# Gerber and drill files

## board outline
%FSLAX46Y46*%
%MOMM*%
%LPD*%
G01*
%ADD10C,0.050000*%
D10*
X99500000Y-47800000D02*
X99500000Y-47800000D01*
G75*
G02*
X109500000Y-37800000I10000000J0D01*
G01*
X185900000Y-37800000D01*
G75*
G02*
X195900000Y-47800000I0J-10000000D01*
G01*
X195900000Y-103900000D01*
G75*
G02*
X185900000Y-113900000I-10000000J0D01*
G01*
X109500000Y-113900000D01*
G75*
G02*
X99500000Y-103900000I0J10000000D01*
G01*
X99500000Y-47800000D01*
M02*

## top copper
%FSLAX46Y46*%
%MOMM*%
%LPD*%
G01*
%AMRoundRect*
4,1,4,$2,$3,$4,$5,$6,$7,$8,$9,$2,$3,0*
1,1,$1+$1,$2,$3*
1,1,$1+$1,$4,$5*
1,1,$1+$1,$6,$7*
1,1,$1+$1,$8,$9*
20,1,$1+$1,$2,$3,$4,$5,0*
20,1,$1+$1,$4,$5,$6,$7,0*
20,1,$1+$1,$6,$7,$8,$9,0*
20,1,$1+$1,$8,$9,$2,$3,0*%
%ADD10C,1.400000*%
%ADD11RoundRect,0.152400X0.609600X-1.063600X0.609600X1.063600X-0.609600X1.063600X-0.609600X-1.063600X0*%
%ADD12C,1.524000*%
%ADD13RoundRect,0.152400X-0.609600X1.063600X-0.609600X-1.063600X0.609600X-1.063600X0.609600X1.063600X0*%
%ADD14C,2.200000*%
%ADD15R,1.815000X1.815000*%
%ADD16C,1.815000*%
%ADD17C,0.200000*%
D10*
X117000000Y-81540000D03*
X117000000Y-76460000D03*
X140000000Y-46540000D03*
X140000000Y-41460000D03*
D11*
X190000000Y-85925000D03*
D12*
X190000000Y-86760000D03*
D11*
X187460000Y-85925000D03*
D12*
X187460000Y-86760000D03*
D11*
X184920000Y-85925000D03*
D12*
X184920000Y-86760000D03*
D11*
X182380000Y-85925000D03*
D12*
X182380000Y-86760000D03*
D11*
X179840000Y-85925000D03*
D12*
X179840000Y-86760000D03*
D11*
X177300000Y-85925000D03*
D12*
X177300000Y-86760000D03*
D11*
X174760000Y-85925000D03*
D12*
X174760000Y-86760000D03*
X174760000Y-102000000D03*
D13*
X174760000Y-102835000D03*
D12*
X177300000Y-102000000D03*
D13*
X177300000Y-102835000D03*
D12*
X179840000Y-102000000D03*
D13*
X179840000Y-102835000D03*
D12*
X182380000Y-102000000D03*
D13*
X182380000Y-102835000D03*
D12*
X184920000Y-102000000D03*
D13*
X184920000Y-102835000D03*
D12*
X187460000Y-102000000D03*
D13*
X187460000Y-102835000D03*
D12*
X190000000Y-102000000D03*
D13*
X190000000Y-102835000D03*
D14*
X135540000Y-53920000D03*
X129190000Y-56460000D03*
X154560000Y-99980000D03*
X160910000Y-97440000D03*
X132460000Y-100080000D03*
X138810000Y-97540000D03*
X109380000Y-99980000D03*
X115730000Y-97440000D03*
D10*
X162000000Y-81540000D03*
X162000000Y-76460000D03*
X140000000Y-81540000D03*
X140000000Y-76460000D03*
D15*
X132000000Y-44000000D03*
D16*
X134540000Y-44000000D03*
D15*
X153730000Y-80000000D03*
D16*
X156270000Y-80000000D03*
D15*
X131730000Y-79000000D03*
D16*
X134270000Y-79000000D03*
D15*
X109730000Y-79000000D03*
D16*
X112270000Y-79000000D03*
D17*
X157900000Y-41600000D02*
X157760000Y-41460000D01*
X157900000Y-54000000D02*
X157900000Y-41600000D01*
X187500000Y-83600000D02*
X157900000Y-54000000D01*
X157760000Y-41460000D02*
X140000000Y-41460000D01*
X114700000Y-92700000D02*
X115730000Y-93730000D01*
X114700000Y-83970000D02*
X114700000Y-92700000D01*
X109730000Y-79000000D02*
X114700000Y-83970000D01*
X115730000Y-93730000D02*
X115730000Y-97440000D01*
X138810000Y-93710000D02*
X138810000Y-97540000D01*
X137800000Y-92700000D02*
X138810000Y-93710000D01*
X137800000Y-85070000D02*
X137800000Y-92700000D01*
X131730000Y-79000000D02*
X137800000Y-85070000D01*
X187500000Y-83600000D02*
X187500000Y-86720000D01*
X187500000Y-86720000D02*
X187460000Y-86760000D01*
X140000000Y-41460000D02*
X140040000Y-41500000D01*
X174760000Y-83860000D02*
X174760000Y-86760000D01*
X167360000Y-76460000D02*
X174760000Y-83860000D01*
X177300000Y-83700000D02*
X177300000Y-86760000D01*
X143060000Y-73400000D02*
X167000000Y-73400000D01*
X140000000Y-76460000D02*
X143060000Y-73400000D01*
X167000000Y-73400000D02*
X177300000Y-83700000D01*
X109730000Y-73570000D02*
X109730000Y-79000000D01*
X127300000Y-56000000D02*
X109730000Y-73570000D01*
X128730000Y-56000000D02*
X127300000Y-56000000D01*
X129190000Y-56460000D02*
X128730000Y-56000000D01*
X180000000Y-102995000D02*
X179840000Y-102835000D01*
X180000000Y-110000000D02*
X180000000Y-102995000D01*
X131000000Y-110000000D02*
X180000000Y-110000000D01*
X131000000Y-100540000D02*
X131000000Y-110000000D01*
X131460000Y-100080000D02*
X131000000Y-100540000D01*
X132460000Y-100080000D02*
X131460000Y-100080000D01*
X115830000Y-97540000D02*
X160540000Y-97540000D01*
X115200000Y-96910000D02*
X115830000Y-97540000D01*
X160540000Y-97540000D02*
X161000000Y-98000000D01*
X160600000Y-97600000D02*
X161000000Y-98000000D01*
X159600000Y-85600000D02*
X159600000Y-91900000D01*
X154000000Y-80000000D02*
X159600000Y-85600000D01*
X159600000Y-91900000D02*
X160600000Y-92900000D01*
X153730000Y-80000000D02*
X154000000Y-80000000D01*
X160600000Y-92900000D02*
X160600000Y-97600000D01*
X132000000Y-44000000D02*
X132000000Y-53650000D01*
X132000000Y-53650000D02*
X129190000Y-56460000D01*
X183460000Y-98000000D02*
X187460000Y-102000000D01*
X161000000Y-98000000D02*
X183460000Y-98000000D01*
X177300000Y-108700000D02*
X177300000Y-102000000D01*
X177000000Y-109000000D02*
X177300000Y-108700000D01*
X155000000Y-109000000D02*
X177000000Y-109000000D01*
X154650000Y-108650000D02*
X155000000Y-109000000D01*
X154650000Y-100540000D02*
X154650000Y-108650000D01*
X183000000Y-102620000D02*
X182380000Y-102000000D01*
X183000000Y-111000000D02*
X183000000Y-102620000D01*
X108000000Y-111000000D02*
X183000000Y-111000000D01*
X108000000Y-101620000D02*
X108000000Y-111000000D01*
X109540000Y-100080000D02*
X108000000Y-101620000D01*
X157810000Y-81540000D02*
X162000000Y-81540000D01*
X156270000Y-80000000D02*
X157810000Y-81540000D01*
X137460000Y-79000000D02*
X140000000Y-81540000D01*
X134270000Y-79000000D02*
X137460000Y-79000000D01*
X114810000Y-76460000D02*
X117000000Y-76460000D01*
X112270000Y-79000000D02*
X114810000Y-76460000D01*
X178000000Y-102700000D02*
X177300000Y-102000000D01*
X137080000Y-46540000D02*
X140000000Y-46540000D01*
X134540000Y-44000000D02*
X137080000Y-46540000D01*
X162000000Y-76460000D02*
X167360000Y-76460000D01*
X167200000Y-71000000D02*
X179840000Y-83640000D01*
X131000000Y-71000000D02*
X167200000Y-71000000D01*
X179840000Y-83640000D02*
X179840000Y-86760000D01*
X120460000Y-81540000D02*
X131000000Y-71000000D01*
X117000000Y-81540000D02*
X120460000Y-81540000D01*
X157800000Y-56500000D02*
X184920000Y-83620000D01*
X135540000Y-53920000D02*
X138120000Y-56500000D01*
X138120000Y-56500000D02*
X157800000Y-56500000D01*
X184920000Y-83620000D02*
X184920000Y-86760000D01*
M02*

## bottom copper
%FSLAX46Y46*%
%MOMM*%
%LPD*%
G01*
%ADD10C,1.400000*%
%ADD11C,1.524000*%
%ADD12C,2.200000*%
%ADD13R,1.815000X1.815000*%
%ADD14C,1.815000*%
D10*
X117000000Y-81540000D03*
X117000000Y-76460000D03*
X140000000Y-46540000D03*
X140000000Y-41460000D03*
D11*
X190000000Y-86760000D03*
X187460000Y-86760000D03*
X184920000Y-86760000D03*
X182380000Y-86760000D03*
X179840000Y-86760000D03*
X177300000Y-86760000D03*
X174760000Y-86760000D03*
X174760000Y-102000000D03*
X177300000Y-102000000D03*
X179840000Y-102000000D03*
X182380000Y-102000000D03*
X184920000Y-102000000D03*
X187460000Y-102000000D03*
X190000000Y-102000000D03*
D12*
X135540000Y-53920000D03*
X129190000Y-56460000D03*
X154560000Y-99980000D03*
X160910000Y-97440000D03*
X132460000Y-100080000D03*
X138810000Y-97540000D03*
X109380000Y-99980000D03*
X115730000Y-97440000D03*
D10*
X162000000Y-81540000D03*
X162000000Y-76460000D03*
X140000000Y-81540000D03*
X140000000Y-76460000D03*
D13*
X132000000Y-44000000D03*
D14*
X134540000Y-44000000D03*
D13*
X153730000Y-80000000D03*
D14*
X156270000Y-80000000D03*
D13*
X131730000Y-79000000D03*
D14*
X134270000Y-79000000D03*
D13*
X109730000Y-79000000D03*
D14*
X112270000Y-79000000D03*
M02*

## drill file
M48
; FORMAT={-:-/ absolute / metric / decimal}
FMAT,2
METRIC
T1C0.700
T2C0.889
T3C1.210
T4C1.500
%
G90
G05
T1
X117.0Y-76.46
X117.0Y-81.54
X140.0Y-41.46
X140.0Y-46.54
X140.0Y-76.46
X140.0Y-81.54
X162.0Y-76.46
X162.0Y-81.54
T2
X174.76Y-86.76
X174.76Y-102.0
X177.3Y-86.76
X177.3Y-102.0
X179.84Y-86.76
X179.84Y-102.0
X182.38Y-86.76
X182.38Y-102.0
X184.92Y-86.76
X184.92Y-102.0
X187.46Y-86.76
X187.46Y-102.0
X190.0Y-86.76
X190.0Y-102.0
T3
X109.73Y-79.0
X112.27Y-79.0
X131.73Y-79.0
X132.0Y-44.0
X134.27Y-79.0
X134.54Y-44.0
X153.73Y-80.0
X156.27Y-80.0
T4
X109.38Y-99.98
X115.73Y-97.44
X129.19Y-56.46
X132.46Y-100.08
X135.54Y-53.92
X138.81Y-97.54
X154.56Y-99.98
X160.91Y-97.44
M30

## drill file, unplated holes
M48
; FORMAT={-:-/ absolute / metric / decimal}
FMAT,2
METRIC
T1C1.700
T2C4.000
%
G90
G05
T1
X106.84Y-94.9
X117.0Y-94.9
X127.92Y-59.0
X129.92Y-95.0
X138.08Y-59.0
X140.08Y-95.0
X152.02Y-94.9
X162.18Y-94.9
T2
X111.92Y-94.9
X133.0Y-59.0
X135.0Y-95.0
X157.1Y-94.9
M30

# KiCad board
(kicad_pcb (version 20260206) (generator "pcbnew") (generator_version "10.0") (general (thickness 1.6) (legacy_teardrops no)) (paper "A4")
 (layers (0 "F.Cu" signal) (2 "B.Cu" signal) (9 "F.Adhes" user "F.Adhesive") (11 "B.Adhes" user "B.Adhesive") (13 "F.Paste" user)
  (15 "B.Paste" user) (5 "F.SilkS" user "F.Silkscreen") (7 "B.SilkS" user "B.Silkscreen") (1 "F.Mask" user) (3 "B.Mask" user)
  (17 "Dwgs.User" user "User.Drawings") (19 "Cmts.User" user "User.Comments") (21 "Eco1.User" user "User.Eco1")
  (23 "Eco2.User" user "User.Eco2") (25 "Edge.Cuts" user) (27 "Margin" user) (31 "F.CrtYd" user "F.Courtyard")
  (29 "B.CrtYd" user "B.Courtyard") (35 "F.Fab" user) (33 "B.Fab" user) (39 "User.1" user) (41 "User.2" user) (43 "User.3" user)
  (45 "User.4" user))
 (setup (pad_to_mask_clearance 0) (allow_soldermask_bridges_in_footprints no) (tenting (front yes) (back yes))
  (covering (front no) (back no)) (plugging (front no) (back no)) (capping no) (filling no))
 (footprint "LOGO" (layer "F.Cu") (at 111.4 50.9)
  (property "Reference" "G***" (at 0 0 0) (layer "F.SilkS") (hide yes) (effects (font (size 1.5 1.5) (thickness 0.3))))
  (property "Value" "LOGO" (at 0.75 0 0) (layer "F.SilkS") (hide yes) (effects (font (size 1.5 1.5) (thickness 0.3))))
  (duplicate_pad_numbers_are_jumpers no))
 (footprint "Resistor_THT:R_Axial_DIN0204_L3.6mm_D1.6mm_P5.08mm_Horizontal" (layer "F.Cu") (at 140 46.54 90)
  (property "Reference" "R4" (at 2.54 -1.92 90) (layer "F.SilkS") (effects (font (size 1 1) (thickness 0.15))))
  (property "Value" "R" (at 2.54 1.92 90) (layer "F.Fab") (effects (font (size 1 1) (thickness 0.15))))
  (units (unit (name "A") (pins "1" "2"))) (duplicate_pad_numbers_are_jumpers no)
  (pad "1" thru_hole circle (at 0 0 90) (size 1.4 1.4) (drill 0.7) (layers "*.Cu" "*.Mask") (remove_unused_layers no) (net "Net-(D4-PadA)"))
  (pad "2" thru_hole circle (at 5.08 0 90) (size 1.4 1.4) (drill 0.7) (layers "*.Cu" "*.Mask") (remove_unused_layers no) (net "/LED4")))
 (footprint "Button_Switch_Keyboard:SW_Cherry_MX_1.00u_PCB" (layer "F.Cu") (at 154.56 99.98 180)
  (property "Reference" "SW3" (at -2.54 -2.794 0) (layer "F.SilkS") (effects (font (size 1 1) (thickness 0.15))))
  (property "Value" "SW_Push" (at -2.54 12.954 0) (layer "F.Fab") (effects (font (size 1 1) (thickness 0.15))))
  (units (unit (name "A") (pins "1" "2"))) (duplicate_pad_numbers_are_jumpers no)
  (pad "" np_thru_hole circle (at -7.62 5.08 180) (size 1.7 1.7) (drill 1.7) (layers "*.Cu" "*.Mask"))
  (pad "" np_thru_hole circle (at -2.54 5.08 180) (size 4 4) (drill 4) (layers "*.Cu" "*.Mask"))
  (pad "" np_thru_hole circle (at 2.54 5.08 180) (size 1.7 1.7) (drill 1.7) (layers "*.Cu" "*.Mask"))
  (pad "1" thru_hole circle (at 0 0 180) (size 2.2 2.2) (drill 1.5) (layers "*.Cu" "*.Mask") (remove_unused_layers no) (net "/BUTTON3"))
  (pad "2" thru_hole circle (at -6.35 2.54 180) (size 2.2 2.2) (drill 1.5) (layers "*.Cu" "*.Mask") (remove_unused_layers no) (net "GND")))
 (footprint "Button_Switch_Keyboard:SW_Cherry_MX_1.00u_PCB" (layer "F.Cu") (at 132.46 100.08 180)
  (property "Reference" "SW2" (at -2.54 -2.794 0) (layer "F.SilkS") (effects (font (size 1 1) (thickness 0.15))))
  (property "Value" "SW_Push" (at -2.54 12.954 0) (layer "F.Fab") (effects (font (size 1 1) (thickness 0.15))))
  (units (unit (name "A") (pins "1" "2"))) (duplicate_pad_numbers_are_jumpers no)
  (pad "" np_thru_hole circle (at -7.62 5.08 180) (size 1.7 1.7) (drill 1.7) (layers "*.Cu" "*.Mask"))
  (pad "" np_thru_hole circle (at -2.54 5.08 180) (size 4 4) (drill 4) (layers "*.Cu" "*.Mask"))
  (pad "" np_thru_hole circle (at 2.54 5.08 180) (size 1.7 1.7) (drill 1.7) (layers "*.Cu" "*.Mask"))
  (pad "1" thru_hole circle (at 0 0 180) (size 2.2 2.2) (drill 1.5) (layers "*.Cu" "*.Mask") (remove_unused_layers no) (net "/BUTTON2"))
  (pad "2" thru_hole circle (at -6.35 2.54 180) (size 2.2 2.2) (drill 1.5) (layers "*.Cu" "*.Mask") (remove_unused_layers no) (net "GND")))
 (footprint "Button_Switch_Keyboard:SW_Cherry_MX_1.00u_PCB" (layer "F.Cu") (at 135.54 53.92)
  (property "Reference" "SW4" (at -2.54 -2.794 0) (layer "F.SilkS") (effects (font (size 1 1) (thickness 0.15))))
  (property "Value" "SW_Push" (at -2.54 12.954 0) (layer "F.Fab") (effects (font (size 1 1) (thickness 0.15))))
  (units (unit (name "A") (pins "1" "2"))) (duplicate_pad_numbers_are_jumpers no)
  (pad "" np_thru_hole circle (at -7.62 5.08) (size 1.7 1.7) (drill 1.7) (layers "*.Cu" "*.Mask"))
  (pad "" np_thru_hole circle (at -2.54 5.08) (size 4 4) (drill 4) (layers "*.Cu" "*.Mask"))
  (pad "" np_thru_hole circle (at 2.54 5.08) (size 1.7 1.7) (drill 1.7) (layers "*.Cu" "*.Mask"))
  (pad "1" thru_hole circle (at 0 0) (size 2.2 2.2) (drill 1.5) (layers "*.Cu" "*.Mask") (remove_unused_layers no) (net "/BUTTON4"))
  (pad "2" thru_hole circle (at -6.35 2.54) (size 2.2 2.2) (drill 1.5) (layers "*.Cu" "*.Mask") (remove_unused_layers no) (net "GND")))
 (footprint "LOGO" (layer "F.Cu") (at 180.3 64.4)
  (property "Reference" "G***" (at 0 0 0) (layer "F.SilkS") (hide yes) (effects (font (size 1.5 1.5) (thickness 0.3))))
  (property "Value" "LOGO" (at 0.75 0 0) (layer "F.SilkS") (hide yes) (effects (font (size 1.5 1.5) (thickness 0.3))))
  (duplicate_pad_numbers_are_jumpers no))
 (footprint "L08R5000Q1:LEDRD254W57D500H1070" (layer "F.Cu") (at 133.27 44)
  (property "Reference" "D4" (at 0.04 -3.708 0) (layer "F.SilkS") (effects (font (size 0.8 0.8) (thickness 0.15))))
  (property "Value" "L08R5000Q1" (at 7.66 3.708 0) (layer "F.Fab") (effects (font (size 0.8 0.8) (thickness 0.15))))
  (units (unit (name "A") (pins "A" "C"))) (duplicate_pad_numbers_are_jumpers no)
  (pad "A" thru_hole circle (at 1.27 0) (size 1.815 1.815) (drill 1.21) (layers "*.Cu" "*.Mask") (remove_unused_layers no)
   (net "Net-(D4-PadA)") (solder_mask_margin 0.102))
  (pad "C" thru_hole rect (at -1.27 0) (size 1.815 1.815) (drill 1.21) (layers "*.Cu" "*.Mask") (remove_unused_layers no) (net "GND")
   (solder_mask_margin 0.102)))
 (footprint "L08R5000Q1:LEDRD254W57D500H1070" (layer "F.Cu") (at 155 80)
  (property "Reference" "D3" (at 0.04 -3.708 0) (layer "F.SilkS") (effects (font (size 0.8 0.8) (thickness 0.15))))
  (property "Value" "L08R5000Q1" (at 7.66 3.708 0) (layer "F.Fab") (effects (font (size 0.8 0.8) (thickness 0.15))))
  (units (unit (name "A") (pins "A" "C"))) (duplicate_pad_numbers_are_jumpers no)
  (pad "A" thru_hole circle (at 1.27 0) (size 1.815 1.815) (drill 1.21) (layers "*.Cu" "*.Mask") (remove_unused_layers no)
   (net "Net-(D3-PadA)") (solder_mask_margin 0.102))
  (pad "C" thru_hole rect (at -1.27 0) (size 1.815 1.815) (drill 1.21) (layers "*.Cu" "*.Mask") (remove_unused_layers no) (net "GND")
   (solder_mask_margin 0.102)))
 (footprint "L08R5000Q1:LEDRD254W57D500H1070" (layer "F.Cu") (at 111 79)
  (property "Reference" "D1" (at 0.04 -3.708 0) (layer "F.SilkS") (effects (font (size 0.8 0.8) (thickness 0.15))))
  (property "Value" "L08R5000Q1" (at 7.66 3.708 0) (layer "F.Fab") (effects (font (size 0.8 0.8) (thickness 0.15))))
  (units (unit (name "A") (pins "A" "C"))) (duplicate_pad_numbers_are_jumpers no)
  (pad "A" thru_hole circle (at 1.27 0) (size 1.815 1.815) (drill 1.21) (layers "*.Cu" "*.Mask") (remove_unused_layers no)
   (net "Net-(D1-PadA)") (solder_mask_margin 0.102))
  (pad "C" thru_hole rect (at -1.27 0) (size 1.815 1.815) (drill 1.21) (layers "*.Cu" "*.Mask") (remove_unused_layers no) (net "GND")
   (solder_mask_margin 0.102)))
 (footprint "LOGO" (layer "F.Cu") (at 170.3 47.5)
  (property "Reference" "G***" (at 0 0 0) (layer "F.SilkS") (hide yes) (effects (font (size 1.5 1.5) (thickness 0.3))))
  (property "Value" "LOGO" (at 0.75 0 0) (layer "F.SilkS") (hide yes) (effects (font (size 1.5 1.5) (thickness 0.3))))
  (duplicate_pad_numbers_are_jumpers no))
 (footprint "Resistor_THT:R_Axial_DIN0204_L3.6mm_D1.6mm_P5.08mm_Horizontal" (layer "F.Cu") (at 117 81.54 90)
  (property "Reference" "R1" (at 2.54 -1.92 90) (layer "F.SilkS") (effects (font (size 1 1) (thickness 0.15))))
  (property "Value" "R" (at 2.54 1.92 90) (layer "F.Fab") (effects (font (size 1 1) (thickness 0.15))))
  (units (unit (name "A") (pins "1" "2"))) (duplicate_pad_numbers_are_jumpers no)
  (pad "1" thru_hole circle (at 0 0 90) (size 1.4 1.4) (drill 0.7) (layers "*.Cu" "*.Mask") (remove_unused_layers no) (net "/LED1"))
  (pad "2" thru_hole circle (at 5.08 0 90) (size 1.4 1.4) (drill 0.7) (layers "*.Cu" "*.Mask") (remove_unused_layers no)
   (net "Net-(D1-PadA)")))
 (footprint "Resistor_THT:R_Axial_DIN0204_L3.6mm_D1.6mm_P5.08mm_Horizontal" (layer "F.Cu") (at 162 81.54 90)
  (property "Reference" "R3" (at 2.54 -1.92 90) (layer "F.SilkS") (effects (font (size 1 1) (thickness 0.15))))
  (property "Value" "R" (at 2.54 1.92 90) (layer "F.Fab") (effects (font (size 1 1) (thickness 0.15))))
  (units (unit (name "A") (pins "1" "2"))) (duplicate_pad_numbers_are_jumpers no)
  (pad "1" thru_hole circle (at 0 0 90) (size 1.4 1.4) (drill 0.7) (layers "*.Cu" "*.Mask") (remove_unused_layers no) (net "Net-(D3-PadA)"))
  (pad "2" thru_hole circle (at 5.08 0 90) (size 1.4 1.4) (drill 0.7) (layers "*.Cu" "*.Mask") (remove_unused_layers no) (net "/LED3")))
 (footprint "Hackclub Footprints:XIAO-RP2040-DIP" (layer "F.Cu") (at 182.38 94.38 -90)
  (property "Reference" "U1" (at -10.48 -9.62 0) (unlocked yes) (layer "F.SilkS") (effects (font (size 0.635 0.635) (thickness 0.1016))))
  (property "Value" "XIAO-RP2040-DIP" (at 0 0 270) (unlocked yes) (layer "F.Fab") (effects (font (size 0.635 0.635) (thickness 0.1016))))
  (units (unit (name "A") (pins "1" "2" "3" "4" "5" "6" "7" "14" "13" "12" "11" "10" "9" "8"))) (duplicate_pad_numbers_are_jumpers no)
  (pad "1" smd roundrect (at -8.455 -7.62 90) (size 2.432 1.524) (layers "F.Cu" "F.Mask") (roundrect_rratio 0.1)
   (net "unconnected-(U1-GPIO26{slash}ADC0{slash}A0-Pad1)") (thermal_bridge_angle 45))
  (pad "1" thru_hole circle (at -7.62 -7.62 90) (size 1.524 1.524) (drill 0.889) (layers "*.Cu" "*.Mask") (remove_unused_layers no)
   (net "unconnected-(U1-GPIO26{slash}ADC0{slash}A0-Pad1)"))
  (pad "2" smd roundrect (at -8.455 -5.08 90) (size 2.432 1.524) (layers "F.Cu" "F.Mask") (roundrect_rratio 0.1) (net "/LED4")
   (thermal_bridge_angle 45))
  (pad "2" thru_hole circle (at -7.62 -5.08 90) (size 1.524 1.524) (drill 0.889) (layers "*.Cu" "*.Mask") (remove_unused_layers no)
   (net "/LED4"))
  (pad "3" smd roundrect (at -8.455 -2.54 90) (size 2.432 1.524) (layers "F.Cu" "F.Mask") (roundrect_rratio 0.1) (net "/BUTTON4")
   (thermal_bridge_angle 45))
  (pad "3" thru_hole circle (at -7.62 -2.54 90) (size 1.524 1.524) (drill 0.889) (layers "*.Cu" "*.Mask") (remove_unused_layers no)
   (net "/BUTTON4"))
  (pad "4" smd roundrect (at -8.455 0 90) (size 2.432 1.524) (layers "F.Cu" "F.Mask") (roundrect_rratio 0.1)
   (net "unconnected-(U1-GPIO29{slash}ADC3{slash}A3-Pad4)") (thermal_bridge_angle 45))
  (pad "4" thru_hole circle (at -7.62 0 90) (size 1.524 1.524) (drill 0.889) (layers "*.Cu" "*.Mask") (remove_unused_layers no)
   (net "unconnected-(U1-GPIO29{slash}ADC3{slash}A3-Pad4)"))
  (pad "5" smd roundrect (at -8.455 2.54 90) (size 2.432 1.524) (layers "F.Cu" "F.Mask") (roundrect_rratio 0.1) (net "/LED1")
   (thermal_bridge_angle 45))
  (pad "5" thru_hole circle (at -7.62 2.54 90) (size 1.524 1.524) (drill 0.889) (layers "*.Cu" "*.Mask") (remove_unused_layers no)
   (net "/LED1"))
  (pad "6" smd roundrect (at -8.455 5.08 90) (size 2.432 1.524) (layers "F.Cu" "F.Mask") (roundrect_rratio 0.1) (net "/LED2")
   (thermal_bridge_angle 45))
  (pad "6" thru_hole circle (at -7.62 5.08 90) (size 1.524 1.524) (drill 0.889) (layers "*.Cu" "*.Mask") (remove_unused_layers no)
   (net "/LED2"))
  (pad "7" smd roundrect (at -8.455 7.62 90) (size 2.432 1.524) (layers "F.Cu" "F.Mask") (roundrect_rratio 0.1) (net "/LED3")
   (thermal_bridge_angle 45))
  (pad "7" thru_hole circle (at -7.62 7.62 90) (size 1.524 1.524) (drill 0.889) (layers "*.Cu" "*.Mask") (remove_unused_layers no)
   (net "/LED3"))
  (pad "8" thru_hole circle (at 7.62 7.62 270) (size 1.524 1.524) (drill 0.889) (layers "*.Cu" "*.Mask") (remove_unused_layers no)
   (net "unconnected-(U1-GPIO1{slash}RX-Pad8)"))
  (pad "8" smd roundrect (at 8.455 7.62 270) (size 2.432 1.524) (layers "F.Cu" "F.Mask") (roundrect_rratio 0.1)
   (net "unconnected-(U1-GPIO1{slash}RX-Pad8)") (thermal_bridge_angle 45))
  (pad "9" thru_hole circle (at 7.62 5.08 270) (size 1.524 1.524) (drill 0.889) (layers "*.Cu" "*.Mask") (remove_unused_layers no)
   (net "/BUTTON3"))
  (pad "9" smd roundrect (at 8.455 5.08 270) (size 2.432 1.524) (layers "F.Cu" "F.Mask") (roundrect_rratio 0.1) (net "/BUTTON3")
   (thermal_bridge_angle 45))
  (pad "10" thru_hole circle (at 7.62 2.54 270) (size 1.524 1.524) (drill 0.889) (layers "*.Cu" "*.Mask") (remove_unused_layers no)
   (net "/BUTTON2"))
  (pad "10" smd roundrect (at 8.455 2.54 270) (size 2.432 1.524) (layers "F.Cu" "F.Mask") (roundrect_rratio 0.1) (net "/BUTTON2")
   (thermal_bridge_angle 45))
  (pad "11" thru_hole circle (at 7.62 0 270) (size 1.524 1.524) (drill 0.889) (layers "*.Cu" "*.Mask") (remove_unused_layers no)
   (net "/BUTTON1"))
  (pad "11" smd roundrect (at 8.455 0 270) (size 2.432 1.524) (layers "F.Cu" "F.Mask") (roundrect_rratio 0.1) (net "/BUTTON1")
   (thermal_bridge_angle 45))
  (pad "12" thru_hole circle (at 7.62 -2.54 270) (size 1.524 1.524) (drill 0.889) (layers "*.Cu" "*.Mask") (remove_unused_layers no)
   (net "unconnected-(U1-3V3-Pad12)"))
  (pad "12" smd roundrect (at 8.455 -2.54 270) (size 2.432 1.524) (layers "F.Cu" "F.Mask") (roundrect_rratio 0.1)
   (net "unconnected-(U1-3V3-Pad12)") (thermal_bridge_angle 45))
  (pad "13" thru_hole circle (at 7.62 -5.08 270) (size 1.524 1.524) (drill 0.889) (layers "*.Cu" "*.Mask") (remove_unused_layers no)
   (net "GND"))
  (pad "13" smd roundrect (at 8.455 -5.08 270) (size 2.432 1.524) (layers "F.Cu" "F.Mask") (roundrect_rratio 0.1) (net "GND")
   (thermal_bridge_angle 45))
  (pad "14" thru_hole circle (at 7.62 -7.62 270) (size 1.524 1.524) (drill 0.889) (layers "*.Cu" "*.Mask") (remove_unused_layers no)
   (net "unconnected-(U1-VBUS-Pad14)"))
  (pad "14" smd roundrect (at 8.455 -7.62 270) (size 2.432 1.524) (layers "F.Cu" "F.Mask") (roundrect_rratio 0.1)
   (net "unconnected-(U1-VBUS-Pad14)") (thermal_bridge_angle 45)))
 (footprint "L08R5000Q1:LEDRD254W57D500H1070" (layer "F.Cu") (at 133 79)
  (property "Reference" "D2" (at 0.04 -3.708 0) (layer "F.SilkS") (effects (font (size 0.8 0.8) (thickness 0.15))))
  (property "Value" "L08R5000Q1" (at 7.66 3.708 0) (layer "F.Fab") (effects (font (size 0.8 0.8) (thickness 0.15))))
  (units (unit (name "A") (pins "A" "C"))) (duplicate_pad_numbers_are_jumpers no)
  (pad "A" thru_hole circle (at 1.27 0) (size 1.815 1.815) (drill 1.21) (layers "*.Cu" "*.Mask") (remove_unused_layers no)
   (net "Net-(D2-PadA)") (solder_mask_margin 0.102))
  (pad "C" thru_hole rect (at -1.27 0) (size 1.815 1.815) (drill 1.21) (layers "*.Cu" "*.Mask") (remove_unused_layers no) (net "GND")
   (solder_mask_margin 0.102)))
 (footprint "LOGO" (layer "F.Cu") (at 182.9 51.3)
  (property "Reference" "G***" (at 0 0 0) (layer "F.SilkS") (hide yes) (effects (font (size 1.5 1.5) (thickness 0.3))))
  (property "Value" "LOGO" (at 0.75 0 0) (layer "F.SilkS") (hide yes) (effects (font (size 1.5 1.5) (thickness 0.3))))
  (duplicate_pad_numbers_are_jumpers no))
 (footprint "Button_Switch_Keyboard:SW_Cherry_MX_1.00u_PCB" (layer "F.Cu") (at 109.38 99.98 180)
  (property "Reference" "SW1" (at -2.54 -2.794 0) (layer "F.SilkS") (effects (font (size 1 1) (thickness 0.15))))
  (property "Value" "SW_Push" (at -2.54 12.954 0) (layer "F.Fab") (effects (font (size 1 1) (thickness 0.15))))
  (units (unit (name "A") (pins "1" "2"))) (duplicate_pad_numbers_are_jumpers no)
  (pad "" np_thru_hole circle (at -7.62 5.08 180) (size 1.7 1.7) (drill 1.7) (layers "*.Cu" "*.Mask"))
  (pad "" np_thru_hole circle (at -2.54 5.08 180) (size 4 4) (drill 4) (layers "*.Cu" "*.Mask"))
  (pad "" np_thru_hole circle (at 2.54 5.08 180) (size 1.7 1.7) (drill 1.7) (layers "*.Cu" "*.Mask"))
  (pad "1" thru_hole circle (at 0 0 180) (size 2.2 2.2) (drill 1.5) (layers "*.Cu" "*.Mask") (remove_unused_layers no) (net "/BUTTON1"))
  (pad "2" thru_hole circle (at -6.35 2.54 180) (size 2.2 2.2) (drill 1.5) (layers "*.Cu" "*.Mask") (remove_unused_layers no) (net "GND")))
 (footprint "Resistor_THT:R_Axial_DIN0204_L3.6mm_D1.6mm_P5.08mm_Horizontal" (layer "F.Cu") (at 140 81.54 90)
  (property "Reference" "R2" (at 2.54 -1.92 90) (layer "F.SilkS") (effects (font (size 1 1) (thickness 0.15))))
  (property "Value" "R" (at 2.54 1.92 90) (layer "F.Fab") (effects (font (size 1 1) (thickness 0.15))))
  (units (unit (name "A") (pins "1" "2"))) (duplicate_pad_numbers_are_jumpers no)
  (pad "1" thru_hole circle (at 0 0 90) (size 1.4 1.4) (drill 0.7) (layers "*.Cu" "*.Mask") (remove_unused_layers no) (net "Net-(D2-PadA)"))
  (pad "2" thru_hole circle (at 5.08 0 90) (size 1.4 1.4) (drill 0.7) (layers "*.Cu" "*.Mask") (remove_unused_layers no) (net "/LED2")))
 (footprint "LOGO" (layer "B.Cu") (at 179.405448 56.483194 180)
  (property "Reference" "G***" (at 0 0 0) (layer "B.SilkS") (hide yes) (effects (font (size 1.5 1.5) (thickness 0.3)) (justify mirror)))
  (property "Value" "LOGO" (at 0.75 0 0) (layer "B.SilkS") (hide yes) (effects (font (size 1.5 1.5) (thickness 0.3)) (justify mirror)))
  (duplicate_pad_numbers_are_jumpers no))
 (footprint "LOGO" (layer "B.Cu") (at 110.818051 63.678154 180)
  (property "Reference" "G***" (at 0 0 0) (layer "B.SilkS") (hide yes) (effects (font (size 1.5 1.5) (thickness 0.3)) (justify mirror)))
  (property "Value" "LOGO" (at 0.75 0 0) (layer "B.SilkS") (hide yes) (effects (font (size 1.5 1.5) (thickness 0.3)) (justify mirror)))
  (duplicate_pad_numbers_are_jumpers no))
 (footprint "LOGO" (layer "B.Cu") (at 111.204014 47.294564 180)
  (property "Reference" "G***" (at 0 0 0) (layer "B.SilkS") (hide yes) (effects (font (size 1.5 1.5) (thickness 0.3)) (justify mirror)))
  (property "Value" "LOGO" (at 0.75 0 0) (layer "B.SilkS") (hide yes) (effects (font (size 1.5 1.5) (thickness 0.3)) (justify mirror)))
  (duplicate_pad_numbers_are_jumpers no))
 (gr_rect (start 99.5 37.8) (end 195.9 113.9) (radius 10) (stroke (width 0.05) (type solid)) (fill no) (layer "Edge.Cuts"))
 (segment (start 114.81 76.46) (end 117 76.46) (width 0.2) (layer "F.Cu") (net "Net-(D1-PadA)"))
 (segment (start 112.27 79) (end 114.81 76.46) (width 0.2) (layer "F.Cu") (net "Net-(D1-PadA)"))
 (segment (start 138.81 93.71) (end 138.81 97.54) (width 0.2) (layer "F.Cu") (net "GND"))
 (segment (start 115.73 93.73) (end 115.73 97.44) (width 0.2) (layer "F.Cu") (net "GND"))
 (segment (start 183.46 98) (end 187.46 102) (width 0.2) (layer "F.Cu") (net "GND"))
 (segment (start 159.6 91.9) (end 160.6 92.9) (width 0.2) (layer "F.Cu") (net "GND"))
 (segment (start 160.6 92.9) (end 160.6 97.6) (width 0.2) (layer "F.Cu") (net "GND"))
 (segment (start 132 44) (end 132 53.65) (width 0.2) (layer "F.Cu") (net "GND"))
 (segment (start 154 80) (end 159.6 85.6) (width 0.2) (layer "F.Cu") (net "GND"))
 (segment (start 129.19 56.46) (end 128.73 56) (width 0.2) (layer "F.Cu") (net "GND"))
 (segment (start 115.2 96.91) (end 115.83 97.54) (width 0.2) (layer "F.Cu") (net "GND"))
 (segment (start 153.73 80) (end 154 80) (width 0.2) (layer "F.Cu") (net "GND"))
 (segment (start 109.73 73.57) (end 109.73 79) (width 0.2) (layer "F.Cu") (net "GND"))
 (segment (start 128.73 56) (end 127.3 56) (width 0.2) (layer "F.Cu") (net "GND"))
 (segment (start 114.7 83.97) (end 114.7 92.7) (width 0.2) (layer "F.Cu") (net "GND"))
 (segment (start 160.54 97.54) (end 161 98) (width 0.2) (layer "F.Cu") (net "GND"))
 (segment (start 159.6 85.6) (end 159.6 91.9) (width 0.2) (layer "F.Cu") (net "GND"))
 (segment (start 109.73 79) (end 114.7 83.97) (width 0.2) (layer "F.Cu") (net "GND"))
 (segment (start 131.73 79) (end 137.8 85.07) (width 0.2) (layer "F.Cu") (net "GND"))
 (segment (start 137.8 92.7) (end 138.81 93.71) (width 0.2) (layer "F.Cu") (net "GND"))
 (segment (start 114.7 92.7) (end 115.73 93.73) (width 0.2) (layer "F.Cu") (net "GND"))
 (segment (start 127.3 56) (end 109.73 73.57) (width 0.2) (layer "F.Cu") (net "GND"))
 (segment (start 160.6 97.6) (end 161 98) (width 0.2) (layer "F.Cu") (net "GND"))
 (segment (start 161 98) (end 183.46 98) (width 0.2) (layer "F.Cu") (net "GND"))
 (segment (start 132 53.65) (end 129.19 56.46) (width 0.2) (layer "F.Cu") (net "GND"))
 (segment (start 115.83 97.54) (end 160.54 97.54) (width 0.2) (layer "F.Cu") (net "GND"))
 (segment (start 137.8 85.07) (end 137.8 92.7) (width 0.2) (layer "F.Cu") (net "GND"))
 (segment (start 137.46 79) (end 140 81.54) (width 0.2) (layer "F.Cu") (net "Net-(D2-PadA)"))
 (segment (start 134.27 79) (end 137.46 79) (width 0.2) (layer "F.Cu") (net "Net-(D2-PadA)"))
 (segment (start 157.81 81.54) (end 162 81.54) (width 0.2) (layer "F.Cu") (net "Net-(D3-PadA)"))
 (segment (start 156.27 80) (end 157.81 81.54) (width 0.2) (layer "F.Cu") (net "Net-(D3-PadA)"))
 (segment (start 134.54 44) (end 137.08 46.54) (width 0.2) (layer "F.Cu") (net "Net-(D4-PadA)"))
 (segment (start 137.08 46.54) (end 140 46.54) (width 0.2) (layer "F.Cu") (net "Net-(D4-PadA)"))
 (segment (start 167.2 71) (end 179.84 83.64) (width 0.2) (layer "F.Cu") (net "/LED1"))
 (segment (start 131 71) (end 167.2 71) (width 0.2) (layer "F.Cu") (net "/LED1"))
 (segment (start 117 81.54) (end 120.46 81.54) (width 0.2) (layer "F.Cu") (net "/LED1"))
 (segment (start 179.84 83.64) (end 179.84 86.76) (width 0.2) (layer "F.Cu") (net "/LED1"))
 (segment (start 120.46 81.54) (end 131 71) (width 0.2) (layer "F.Cu") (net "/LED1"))
 (segment (start 140 76.46) (end 143.06 73.4) (width 0.2) (layer "F.Cu") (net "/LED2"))
 (segment (start 143.06 73.4) (end 167 73.4) (width 0.2) (layer "F.Cu") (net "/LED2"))
 (segment (start 177.3 83.7) (end 177.3 86.76) (width 0.2) (layer "F.Cu") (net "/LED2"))
 (segment (start 167 73.4) (end 177.3 83.7) (width 0.2) (layer "F.Cu") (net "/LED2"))
 (segment (start 162 76.46) (end 167.36 76.46) (width 0.2) (layer "F.Cu") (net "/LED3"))
 (segment (start 167.36 76.46) (end 174.76 83.86) (width 0.2) (layer "F.Cu") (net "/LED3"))
 (segment (start 174.76 83.86) (end 174.76 86.76) (width 0.2) (layer "F.Cu") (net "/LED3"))
 (segment (start 187.5 83.6) (end 187.5 86.72) (width 0.2) (layer "F.Cu") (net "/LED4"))
 (segment (start 187.5 83.6) (end 157.9 54) (width 0.2) (layer "F.Cu") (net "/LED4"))
 (segment (start 187.5 86.72) (end 187.46 86.76) (width 0.2) (layer "F.Cu") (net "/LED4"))
 (segment (start 140 41.46) (end 140.04 41.5) (width 0.2) (layer "F.Cu") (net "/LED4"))
 (segment (start 157.9 41.6) (end 157.76 41.46) (width 0.2) (layer "F.Cu") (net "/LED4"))
 (segment (start 157.76 41.46) (end 140 41.46) (width 0.2) (layer "F.Cu") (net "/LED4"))
 (segment (start 157.9 54) (end 157.9 41.6) (width 0.2) (layer "F.Cu") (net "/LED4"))
 (segment (start 109.54 100.08) (end 108 101.62) (width 0.2) (layer "F.Cu") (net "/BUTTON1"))
 (segment (start 108 101.62) (end 108 111) (width 0.2) (layer "F.Cu") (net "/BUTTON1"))
 (segment (start 108 111) (end 183 111) (width 0.2) (layer "F.Cu") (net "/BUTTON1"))
 (segment (start 183 102.62) (end 182.38 102) (width 0.2) (layer "F.Cu") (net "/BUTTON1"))
 (segment (start 183 111) (end 183 102.62) (width 0.2) (layer "F.Cu") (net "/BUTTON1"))
 (segment (start 131 110) (end 180 110) (width 0.2) (layer "F.Cu") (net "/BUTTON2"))
 (segment (start 131.46 100.08) (end 131 100.54) (width 0.2) (layer "F.Cu") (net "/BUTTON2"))
 (segment (start 131 100.54) (end 131 110) (width 0.2) (layer "F.Cu") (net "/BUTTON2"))
 (segment (start 132.46 100.08) (end 131.46 100.08) (width 0.2) (layer "F.Cu") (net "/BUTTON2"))
 (segment (start 180 110) (end 180 102.995) (width 0.2) (layer "F.Cu") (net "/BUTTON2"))
 (segment (start 180 102.995) (end 179.84 102.835) (width 0.2) (layer "F.Cu") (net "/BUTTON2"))
 (segment (start 155 109) (end 177 109) (width 0.2) (layer "F.Cu") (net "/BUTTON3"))
 (segment (start 154.65 108.65) (end 155 109) (width 0.2) (layer "F.Cu") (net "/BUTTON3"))
 (segment (start 178 102.7) (end 177.3 102) (width 0.2) (layer "F.Cu") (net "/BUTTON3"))
 (segment (start 177.3 108.7) (end 177.3 102) (width 0.2) (layer "F.Cu") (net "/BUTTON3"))
 (segment (start 177 109) (end 177.3 108.7) (width 0.2) (layer "F.Cu") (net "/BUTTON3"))
 (segment (start 154.65 100.54) (end 154.65 108.65) (width 0.2) (layer "F.Cu") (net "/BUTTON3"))
 (segment (start 184.92 83.62) (end 184.92 86.76) (width 0.2) (layer "F.Cu") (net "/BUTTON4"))
 (segment (start 135.54 53.92) (end 138.12 56.5) (width 0.2) (layer "F.Cu") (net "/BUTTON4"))
 (segment (start 138.12 56.5) (end 157.8 56.5) (width 0.2) (layer "F.Cu") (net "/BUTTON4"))
 (segment (start 157.8 56.5) (end 184.92 83.62) (width 0.2) (layer "F.Cu") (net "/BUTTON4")))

